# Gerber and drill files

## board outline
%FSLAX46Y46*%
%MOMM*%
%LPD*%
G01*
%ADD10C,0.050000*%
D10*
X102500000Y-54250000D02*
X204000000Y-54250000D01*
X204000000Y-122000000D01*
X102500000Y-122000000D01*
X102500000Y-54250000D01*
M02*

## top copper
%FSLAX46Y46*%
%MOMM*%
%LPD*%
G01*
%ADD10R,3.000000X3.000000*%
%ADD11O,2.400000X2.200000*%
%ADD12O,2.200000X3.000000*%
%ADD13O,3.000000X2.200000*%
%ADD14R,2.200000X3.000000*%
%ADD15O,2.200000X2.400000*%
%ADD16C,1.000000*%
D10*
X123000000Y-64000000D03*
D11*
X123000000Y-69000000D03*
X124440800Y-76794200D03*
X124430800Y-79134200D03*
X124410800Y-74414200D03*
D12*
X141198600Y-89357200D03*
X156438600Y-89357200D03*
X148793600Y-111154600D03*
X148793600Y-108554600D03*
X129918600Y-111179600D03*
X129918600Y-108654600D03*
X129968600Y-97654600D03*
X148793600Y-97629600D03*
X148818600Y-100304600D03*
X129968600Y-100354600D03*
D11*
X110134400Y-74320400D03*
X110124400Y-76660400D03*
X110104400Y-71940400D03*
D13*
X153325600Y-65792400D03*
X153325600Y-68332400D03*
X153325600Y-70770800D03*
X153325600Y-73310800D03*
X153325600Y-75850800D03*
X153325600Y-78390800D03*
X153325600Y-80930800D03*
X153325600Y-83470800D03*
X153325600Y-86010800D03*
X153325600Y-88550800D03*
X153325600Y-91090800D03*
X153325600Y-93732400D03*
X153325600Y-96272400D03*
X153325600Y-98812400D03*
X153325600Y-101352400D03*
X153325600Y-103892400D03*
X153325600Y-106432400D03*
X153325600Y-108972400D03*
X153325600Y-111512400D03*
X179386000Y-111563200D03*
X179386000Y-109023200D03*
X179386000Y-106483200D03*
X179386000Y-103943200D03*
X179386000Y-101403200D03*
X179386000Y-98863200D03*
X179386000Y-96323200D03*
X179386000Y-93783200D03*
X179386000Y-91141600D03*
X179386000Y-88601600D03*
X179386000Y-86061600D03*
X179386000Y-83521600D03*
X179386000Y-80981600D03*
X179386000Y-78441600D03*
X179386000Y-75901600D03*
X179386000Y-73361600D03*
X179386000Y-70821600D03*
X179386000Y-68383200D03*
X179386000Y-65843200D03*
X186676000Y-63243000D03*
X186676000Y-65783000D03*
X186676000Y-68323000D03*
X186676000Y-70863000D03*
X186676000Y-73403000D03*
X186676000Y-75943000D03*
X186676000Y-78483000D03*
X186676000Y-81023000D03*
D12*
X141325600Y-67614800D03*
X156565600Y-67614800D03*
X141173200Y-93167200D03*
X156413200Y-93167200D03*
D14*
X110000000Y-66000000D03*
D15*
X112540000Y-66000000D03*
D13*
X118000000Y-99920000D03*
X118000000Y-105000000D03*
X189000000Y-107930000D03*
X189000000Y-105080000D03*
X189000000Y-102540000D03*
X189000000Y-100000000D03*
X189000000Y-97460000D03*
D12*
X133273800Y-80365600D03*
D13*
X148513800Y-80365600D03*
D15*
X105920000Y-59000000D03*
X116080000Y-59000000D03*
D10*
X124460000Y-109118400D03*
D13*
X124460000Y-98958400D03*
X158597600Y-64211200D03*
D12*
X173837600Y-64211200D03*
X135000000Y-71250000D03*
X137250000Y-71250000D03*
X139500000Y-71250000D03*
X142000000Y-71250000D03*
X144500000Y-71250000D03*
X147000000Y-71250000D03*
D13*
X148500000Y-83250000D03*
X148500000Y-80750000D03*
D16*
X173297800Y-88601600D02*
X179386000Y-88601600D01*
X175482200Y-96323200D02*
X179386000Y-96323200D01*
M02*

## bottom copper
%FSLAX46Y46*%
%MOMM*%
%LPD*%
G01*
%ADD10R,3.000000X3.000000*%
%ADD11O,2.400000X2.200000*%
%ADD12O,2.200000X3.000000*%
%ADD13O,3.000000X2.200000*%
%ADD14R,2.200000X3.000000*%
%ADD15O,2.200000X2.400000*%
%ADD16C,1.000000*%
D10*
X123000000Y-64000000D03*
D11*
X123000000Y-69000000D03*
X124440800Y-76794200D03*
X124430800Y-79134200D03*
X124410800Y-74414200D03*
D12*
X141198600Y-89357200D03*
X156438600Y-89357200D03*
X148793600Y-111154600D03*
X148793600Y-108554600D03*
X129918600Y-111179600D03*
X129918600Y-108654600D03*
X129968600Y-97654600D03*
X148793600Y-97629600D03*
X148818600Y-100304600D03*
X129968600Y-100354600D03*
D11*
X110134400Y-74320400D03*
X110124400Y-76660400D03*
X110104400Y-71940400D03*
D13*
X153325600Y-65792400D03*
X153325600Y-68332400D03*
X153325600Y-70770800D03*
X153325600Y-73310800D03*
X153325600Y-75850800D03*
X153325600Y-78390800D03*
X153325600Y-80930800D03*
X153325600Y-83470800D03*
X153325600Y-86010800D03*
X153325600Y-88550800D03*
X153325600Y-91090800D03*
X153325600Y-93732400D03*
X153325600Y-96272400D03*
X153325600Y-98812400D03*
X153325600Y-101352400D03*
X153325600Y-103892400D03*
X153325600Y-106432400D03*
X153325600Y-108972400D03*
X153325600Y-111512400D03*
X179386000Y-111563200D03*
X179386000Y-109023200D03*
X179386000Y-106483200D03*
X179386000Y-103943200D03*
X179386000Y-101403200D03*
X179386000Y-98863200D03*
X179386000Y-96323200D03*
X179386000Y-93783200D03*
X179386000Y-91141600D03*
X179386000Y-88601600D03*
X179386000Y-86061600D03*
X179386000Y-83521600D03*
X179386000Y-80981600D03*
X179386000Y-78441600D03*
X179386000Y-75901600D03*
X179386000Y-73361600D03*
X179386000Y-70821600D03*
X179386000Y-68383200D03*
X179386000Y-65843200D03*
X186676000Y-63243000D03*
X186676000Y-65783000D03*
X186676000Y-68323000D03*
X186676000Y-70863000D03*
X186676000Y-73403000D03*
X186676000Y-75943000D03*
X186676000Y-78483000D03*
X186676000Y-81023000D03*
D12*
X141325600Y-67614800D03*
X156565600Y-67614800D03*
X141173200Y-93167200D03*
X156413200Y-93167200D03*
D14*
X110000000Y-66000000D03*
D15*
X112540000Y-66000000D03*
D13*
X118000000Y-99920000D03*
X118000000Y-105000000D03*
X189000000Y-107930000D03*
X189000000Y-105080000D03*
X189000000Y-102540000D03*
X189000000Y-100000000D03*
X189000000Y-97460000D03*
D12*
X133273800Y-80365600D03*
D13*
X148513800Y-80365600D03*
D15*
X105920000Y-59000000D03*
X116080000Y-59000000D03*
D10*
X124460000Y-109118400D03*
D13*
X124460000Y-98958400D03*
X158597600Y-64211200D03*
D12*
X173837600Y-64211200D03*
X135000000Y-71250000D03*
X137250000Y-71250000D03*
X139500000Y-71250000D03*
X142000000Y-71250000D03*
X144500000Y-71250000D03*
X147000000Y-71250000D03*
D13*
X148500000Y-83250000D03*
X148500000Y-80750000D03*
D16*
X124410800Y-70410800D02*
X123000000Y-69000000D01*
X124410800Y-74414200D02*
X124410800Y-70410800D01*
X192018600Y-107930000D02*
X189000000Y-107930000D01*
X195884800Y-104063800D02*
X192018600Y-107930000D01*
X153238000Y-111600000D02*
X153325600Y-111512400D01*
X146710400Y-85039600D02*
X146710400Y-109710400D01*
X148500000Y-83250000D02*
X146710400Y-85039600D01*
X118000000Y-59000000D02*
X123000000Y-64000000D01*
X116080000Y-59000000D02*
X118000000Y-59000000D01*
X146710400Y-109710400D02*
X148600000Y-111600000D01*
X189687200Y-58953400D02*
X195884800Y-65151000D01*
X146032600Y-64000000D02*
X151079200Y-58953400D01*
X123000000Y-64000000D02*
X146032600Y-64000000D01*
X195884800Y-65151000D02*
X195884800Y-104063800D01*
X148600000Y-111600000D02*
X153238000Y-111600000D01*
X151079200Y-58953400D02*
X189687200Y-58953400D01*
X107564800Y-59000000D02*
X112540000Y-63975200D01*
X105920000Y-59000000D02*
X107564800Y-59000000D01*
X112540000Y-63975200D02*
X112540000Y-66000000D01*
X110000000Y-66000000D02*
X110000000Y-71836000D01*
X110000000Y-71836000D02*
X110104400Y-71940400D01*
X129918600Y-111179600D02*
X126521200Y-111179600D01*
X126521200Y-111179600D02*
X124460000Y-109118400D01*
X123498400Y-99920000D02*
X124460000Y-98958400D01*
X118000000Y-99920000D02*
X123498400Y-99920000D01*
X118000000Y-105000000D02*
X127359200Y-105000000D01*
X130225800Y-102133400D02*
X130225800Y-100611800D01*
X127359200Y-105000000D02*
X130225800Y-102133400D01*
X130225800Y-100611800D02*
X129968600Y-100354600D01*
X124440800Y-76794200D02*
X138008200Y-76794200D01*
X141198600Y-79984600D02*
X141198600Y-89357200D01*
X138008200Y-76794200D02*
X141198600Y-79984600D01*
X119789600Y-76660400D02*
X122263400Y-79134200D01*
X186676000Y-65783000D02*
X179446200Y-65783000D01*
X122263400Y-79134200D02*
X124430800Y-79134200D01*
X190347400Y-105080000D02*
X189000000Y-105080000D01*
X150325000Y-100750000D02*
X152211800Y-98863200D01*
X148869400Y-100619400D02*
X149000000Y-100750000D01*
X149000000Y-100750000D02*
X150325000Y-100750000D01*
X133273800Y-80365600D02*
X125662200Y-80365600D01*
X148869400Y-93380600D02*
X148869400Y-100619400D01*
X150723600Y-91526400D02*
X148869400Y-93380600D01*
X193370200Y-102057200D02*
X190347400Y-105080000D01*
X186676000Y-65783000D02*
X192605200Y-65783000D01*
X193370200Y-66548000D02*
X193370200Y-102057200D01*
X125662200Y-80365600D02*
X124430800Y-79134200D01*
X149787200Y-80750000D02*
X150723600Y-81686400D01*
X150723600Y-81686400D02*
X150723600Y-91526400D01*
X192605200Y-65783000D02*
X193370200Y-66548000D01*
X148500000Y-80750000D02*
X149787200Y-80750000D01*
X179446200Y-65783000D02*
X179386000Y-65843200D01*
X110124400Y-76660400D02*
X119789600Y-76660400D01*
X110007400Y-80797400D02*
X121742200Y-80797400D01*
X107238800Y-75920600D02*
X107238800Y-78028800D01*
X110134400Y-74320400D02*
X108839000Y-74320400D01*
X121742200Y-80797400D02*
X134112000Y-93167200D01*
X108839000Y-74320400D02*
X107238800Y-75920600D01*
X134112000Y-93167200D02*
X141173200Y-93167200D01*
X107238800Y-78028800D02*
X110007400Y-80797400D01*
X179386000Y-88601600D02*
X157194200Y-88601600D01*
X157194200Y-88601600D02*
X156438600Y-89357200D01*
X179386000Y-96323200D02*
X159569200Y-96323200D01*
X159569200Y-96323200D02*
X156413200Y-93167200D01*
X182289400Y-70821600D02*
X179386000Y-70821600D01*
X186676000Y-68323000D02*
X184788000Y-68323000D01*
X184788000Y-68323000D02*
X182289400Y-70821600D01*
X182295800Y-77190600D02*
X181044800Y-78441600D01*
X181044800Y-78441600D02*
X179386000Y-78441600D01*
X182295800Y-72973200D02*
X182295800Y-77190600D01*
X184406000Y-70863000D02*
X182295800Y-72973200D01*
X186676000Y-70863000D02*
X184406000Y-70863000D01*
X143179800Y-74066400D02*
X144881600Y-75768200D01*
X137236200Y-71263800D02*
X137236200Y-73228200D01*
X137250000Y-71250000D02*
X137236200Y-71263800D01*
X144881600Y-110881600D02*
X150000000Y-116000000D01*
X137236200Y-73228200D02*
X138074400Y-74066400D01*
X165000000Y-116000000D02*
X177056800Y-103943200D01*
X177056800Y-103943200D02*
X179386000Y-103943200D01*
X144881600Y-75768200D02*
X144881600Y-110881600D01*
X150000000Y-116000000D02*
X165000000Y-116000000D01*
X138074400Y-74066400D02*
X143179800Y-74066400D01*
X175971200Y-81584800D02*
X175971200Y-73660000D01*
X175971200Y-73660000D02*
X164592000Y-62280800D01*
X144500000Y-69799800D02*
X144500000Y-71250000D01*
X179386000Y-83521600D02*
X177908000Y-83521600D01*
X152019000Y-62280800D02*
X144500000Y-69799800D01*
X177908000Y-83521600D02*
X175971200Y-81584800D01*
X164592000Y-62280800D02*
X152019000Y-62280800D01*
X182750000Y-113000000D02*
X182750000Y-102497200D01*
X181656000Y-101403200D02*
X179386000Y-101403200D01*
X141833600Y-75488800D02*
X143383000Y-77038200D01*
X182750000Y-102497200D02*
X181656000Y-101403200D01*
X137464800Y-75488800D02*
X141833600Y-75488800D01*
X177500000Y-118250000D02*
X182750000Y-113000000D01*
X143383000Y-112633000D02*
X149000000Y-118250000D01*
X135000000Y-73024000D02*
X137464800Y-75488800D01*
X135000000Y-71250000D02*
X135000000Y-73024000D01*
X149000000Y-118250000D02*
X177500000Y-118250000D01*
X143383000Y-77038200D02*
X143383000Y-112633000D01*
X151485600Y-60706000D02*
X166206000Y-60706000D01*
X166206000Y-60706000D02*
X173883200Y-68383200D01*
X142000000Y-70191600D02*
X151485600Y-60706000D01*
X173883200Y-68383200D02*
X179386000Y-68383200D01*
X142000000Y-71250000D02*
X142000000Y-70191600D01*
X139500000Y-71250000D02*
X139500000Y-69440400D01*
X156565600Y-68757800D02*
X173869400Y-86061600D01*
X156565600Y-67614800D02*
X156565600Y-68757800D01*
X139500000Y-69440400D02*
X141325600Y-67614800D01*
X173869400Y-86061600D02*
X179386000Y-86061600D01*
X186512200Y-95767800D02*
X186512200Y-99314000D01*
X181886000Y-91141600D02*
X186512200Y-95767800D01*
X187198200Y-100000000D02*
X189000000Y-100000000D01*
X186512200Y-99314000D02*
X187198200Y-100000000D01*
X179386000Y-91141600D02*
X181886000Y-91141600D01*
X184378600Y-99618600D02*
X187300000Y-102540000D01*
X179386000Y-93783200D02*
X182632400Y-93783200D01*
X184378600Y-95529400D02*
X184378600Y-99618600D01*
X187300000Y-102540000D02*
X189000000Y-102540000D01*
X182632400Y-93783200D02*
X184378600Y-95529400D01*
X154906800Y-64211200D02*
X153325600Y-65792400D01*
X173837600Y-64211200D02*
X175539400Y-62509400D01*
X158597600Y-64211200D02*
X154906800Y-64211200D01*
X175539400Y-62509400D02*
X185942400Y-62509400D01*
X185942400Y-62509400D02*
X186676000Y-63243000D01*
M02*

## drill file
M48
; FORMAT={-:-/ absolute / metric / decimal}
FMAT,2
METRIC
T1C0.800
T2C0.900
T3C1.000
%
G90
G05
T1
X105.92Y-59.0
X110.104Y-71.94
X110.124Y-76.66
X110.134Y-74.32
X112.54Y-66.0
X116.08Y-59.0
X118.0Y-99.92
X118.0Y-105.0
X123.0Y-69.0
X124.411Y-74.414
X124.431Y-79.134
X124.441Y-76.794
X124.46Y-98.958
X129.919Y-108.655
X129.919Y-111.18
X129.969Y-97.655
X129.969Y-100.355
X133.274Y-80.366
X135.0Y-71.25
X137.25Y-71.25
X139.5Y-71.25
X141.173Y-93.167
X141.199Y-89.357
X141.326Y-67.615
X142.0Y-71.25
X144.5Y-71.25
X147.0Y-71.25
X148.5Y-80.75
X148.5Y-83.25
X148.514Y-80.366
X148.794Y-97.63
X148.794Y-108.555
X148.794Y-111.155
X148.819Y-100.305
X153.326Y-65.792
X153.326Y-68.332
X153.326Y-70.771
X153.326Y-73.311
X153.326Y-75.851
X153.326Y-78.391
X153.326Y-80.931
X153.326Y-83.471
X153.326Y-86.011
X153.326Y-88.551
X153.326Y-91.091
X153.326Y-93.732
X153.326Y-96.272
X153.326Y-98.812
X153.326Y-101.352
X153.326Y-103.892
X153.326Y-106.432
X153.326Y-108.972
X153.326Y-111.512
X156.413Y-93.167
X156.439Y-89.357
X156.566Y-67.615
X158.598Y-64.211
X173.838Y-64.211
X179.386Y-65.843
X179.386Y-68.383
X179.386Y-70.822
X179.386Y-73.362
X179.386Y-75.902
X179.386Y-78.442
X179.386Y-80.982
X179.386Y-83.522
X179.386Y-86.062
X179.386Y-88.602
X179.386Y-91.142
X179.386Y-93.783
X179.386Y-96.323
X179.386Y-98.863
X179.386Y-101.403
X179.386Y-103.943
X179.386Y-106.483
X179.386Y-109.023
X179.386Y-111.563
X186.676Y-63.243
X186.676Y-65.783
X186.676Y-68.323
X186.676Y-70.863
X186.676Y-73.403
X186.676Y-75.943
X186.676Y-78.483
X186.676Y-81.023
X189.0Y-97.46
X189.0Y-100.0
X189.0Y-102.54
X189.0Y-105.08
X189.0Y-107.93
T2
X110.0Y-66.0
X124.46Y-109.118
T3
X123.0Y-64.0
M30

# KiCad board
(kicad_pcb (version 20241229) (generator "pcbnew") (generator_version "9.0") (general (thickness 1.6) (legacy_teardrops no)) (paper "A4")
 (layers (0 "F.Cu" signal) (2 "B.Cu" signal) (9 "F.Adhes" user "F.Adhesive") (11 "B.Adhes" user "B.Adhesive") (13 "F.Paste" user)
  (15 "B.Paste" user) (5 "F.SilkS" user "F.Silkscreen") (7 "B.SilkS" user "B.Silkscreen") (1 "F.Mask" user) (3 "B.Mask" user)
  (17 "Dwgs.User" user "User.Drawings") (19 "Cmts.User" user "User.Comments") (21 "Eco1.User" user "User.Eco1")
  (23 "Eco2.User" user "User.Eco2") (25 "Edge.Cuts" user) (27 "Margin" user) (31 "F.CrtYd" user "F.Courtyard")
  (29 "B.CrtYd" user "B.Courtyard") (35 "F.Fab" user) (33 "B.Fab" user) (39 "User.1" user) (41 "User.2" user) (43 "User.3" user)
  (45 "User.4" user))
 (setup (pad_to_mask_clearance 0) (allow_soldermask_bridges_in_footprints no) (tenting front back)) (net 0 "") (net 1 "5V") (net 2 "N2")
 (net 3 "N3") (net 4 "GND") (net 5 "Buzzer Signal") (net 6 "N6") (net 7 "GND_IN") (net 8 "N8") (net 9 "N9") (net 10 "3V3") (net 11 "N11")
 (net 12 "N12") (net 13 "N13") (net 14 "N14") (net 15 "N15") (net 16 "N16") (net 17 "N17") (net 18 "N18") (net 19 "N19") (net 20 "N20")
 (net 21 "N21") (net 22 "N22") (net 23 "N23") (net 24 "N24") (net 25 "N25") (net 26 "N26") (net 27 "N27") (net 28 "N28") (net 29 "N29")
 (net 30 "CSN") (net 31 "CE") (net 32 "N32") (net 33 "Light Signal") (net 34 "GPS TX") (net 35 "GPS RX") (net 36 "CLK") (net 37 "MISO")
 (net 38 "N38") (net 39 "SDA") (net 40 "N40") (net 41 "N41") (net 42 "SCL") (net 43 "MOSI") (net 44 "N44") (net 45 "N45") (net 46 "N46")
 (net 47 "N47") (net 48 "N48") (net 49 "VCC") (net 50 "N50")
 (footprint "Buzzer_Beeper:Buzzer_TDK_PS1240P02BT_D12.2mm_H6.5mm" (layer "F.Cu") (at 123 64 -90)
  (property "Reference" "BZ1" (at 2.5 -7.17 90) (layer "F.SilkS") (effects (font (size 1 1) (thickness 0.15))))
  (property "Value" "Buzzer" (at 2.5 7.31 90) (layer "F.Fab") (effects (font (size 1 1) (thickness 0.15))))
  (pad "1" thru_hole rect (at 0 0 270) (size 3 3) (drill 1) (layers "*.Cu" "*.Mask") (remove_unused_layers no) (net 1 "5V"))
  (pad "2" thru_hole oval (at 5 0) (size 2.4 2.2) (drill 0.8) (layers "*.Cu" "*.Mask") (remove_unused_layers no) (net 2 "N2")
   (thermal_bridge_angle 45)))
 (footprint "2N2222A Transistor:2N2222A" (layer "F.Cu") (at 125.7808 76.7842 -90)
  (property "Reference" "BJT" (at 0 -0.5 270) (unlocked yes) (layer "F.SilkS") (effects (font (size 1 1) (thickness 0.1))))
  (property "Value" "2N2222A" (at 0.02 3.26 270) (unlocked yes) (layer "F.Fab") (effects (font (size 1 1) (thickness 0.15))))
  (pad "1" thru_hole oval (at 0.01 1.34) (size 2.4 2.2) (drill 0.8) (layers "*.Cu" "*.Mask") (remove_unused_layers no) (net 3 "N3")
   (thermal_bridge_angle 45))
  (pad "2" thru_hole oval (at 2.35 1.35) (size 2.4 2.2) (drill 0.8) (layers "*.Cu" "*.Mask") (remove_unused_layers no) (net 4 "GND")
   (thermal_bridge_angle 45))
  (pad "3" thru_hole oval (at -2.37 1.37) (size 2.4 2.2) (drill 0.8) (layers "*.Cu" "*.Mask") (remove_unused_layers no) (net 2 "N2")
   (thermal_bridge_angle 45)))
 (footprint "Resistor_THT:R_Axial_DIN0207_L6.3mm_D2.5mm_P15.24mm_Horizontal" (layer "F.Cu") (at 141.1986 89.3572)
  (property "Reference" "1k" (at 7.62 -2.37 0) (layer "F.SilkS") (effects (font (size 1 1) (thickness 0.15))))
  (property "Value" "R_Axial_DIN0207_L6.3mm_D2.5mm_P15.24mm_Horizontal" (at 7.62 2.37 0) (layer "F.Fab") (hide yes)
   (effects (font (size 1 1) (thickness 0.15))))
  (pad "1" thru_hole oval (at 0 0) (size 2.2 3) (drill 0.8) (layers "*.Cu" "*.Mask") (remove_unused_layers no) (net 3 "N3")
   (thermal_bridge_angle 45))
  (pad "2" thru_hole oval (at 15.24 0) (size 2.2 3) (drill 0.8) (layers "*.Cu" "*.Mask") (remove_unused_layers no) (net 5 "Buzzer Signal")
   (thermal_bridge_angle 45)))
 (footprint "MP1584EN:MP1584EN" (layer "F.Cu") (at 150.8936 113.4546 180)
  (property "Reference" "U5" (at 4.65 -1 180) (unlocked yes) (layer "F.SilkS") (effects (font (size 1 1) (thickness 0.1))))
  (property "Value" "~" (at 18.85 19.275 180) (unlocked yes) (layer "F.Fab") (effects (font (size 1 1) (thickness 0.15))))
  (pad "1" thru_hole oval (at 2.1 2.3 180) (size 2.2 3) (drill 0.8) (layers "*.Cu" "*.Mask") (remove_unused_layers no) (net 1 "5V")
   (thermal_bridge_angle 45))
  (pad "2" thru_hole oval (at 2.1 4.9 180) (size 2.2 3) (drill 0.8) (layers "*.Cu" "*.Mask") (remove_unused_layers no)
   (thermal_bridge_angle 45))
  (pad "3" thru_hole oval (at 20.975 2.275 180) (size 2.2 3) (drill 0.8) (layers "*.Cu" "*.Mask") (remove_unused_layers no) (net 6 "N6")
   (thermal_bridge_angle 45))
  (pad "4" thru_hole oval (at 20.975 4.8 180) (size 2.2 3) (drill 0.8) (layers "*.Cu" "*.Mask") (remove_unused_layers no)
   (thermal_bridge_angle 45))
  (pad "5" thru_hole oval (at 20.925 15.8 180) (size 2.2 3) (drill 0.8) (layers "*.Cu" "*.Mask") (remove_unused_layers no)
   (thermal_bridge_angle 45))
  (pad "6" thru_hole oval (at 2.1 15.825 180) (size 2.2 3) (drill 0.8) (layers "*.Cu" "*.Mask") (remove_unused_layers no)
   (thermal_bridge_angle 45))
  (pad "7" thru_hole oval (at 2.075 13.15 180) (size 2.2 3) (drill 0.8) (layers "*.Cu" "*.Mask") (remove_unused_layers no) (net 4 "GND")
   (thermal_bridge_angle 45))
  (pad "8" thru_hole oval (at 20.925 13.1 180) (size 2.2 3) (drill 0.8) (layers "*.Cu" "*.Mask") (remove_unused_layers no) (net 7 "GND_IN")
   (thermal_bridge_angle 45)))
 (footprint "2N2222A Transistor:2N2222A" (layer "F.Cu") (at 111.4744 74.3104 -90)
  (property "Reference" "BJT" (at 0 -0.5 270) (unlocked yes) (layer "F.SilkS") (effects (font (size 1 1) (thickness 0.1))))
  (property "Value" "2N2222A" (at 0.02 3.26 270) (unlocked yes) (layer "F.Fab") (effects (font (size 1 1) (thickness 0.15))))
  (pad "1" thru_hole oval (at 0.01 1.34) (size 2.4 2.2) (drill 0.8) (layers "*.Cu" "*.Mask") (remove_unused_layers no) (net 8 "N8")
   (thermal_bridge_angle 45))
  (pad "2" thru_hole oval (at 2.35 1.35) (size 2.4 2.2) (drill 0.8) (layers "*.Cu" "*.Mask") (remove_unused_layers no) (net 4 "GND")
   (thermal_bridge_angle 45))
  (pad "3" thru_hole oval (at -2.37 1.37) (size 2.4 2.2) (drill 0.8) (layers "*.Cu" "*.Mask") (remove_unused_layers no) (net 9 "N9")
   (thermal_bridge_angle 45)))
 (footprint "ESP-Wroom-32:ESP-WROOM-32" (layer "F.Cu") (at 153.986 61.4236)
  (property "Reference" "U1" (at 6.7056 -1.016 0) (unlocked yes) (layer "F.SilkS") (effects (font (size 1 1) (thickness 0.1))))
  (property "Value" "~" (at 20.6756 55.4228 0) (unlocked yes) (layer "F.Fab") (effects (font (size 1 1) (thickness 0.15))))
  (pad "1" thru_hole oval (at -0.6604 4.3688) (size 3 2.2) (drill 0.8) (layers "*.Cu" "*.Mask") (remove_unused_layers no) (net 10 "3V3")
   (thermal_bridge_angle 45))
  (pad "2" thru_hole oval (at -0.6604 6.9088) (size 3 2.2) (drill 0.8) (layers "*.Cu" "*.Mask") (remove_unused_layers no) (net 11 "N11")
   (thermal_bridge_angle 45))
  (pad "3" thru_hole oval (at -0.6604 9.3472) (size 3 2.2) (drill 0.8) (layers "*.Cu" "*.Mask") (remove_unused_layers no) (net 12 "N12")
   (thermal_bridge_angle 45))
  (pad "4" thru_hole oval (at -0.6604 11.8872) (size 3 2.2) (drill 0.8) (layers "*.Cu" "*.Mask") (remove_unused_layers no) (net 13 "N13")
   (thermal_bridge_angle 45))
  (pad "5" thru_hole oval (at -0.6604 14.4272) (size 3 2.2) (drill 0.8) (layers "*.Cu" "*.Mask") (remove_unused_layers no) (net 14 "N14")
   (thermal_bridge_angle 45))
  (pad "6" thru_hole oval (at -0.6604 16.9672) (size 3 2.2) (drill 0.8) (layers "*.Cu" "*.Mask") (remove_unused_layers no) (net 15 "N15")
   (thermal_bridge_angle 45))
  (pad "7" thru_hole oval (at -0.6604 19.5072) (size 3 2.2) (drill 0.8) (layers "*.Cu" "*.Mask") (remove_unused_layers no) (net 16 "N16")
   (thermal_bridge_angle 45))
  (pad "8" thru_hole oval (at -0.6604 22.0472) (size 3 2.2) (drill 0.8) (layers "*.Cu" "*.Mask") (remove_unused_layers no) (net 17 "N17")
   (thermal_bridge_angle 45))
  (pad "9" thru_hole oval (at -0.6604 24.5872) (size 3 2.2) (drill 0.8) (layers "*.Cu" "*.Mask") (remove_unused_layers no) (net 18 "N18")
   (thermal_bridge_angle 45))
  (pad "10" thru_hole oval (at -0.6604 27.1272) (size 3 2.2) (drill 0.8) (layers "*.Cu" "*.Mask") (remove_unused_layers no) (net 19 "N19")
   (thermal_bridge_angle 45))
  (pad "11" thru_hole oval (at -0.6604 29.6672) (size 3 2.2) (drill 0.8) (layers "*.Cu" "*.Mask") (remove_unused_layers no) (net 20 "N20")
   (thermal_bridge_angle 45))
  (pad "12" thru_hole oval (at -0.6604 32.3088) (size 3 2.2) (drill 0.8) (layers "*.Cu" "*.Mask") (remove_unused_layers no) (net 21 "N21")
   (thermal_bridge_angle 45))
  (pad "13" thru_hole oval (at -0.6604 34.8488) (size 3 2.2) (drill 0.8) (layers "*.Cu" "*.Mask") (remove_unused_layers no) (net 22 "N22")
   (thermal_bridge_angle 45))
  (pad "14" thru_hole oval (at -0.6604 37.3888) (size 3 2.2) (drill 0.8) (layers "*.Cu" "*.Mask") (remove_unused_layers no) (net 4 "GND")
   (thermal_bridge_angle 45))
  (pad "15" thru_hole oval (at -0.6604 39.9288) (size 3 2.2) (drill 0.8) (layers "*.Cu" "*.Mask") (remove_unused_layers no) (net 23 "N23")
   (thermal_bridge_angle 45))
  (pad "16" thru_hole oval (at -0.6604 42.4688) (size 3 2.2) (drill 0.8) (layers "*.Cu" "*.Mask") (remove_unused_layers no) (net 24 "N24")
   (thermal_bridge_angle 45))
  (pad "17" thru_hole oval (at -0.6604 45.0088) (size 3 2.2) (drill 0.8) (layers "*.Cu" "*.Mask") (remove_unused_layers no) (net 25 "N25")
   (thermal_bridge_angle 45))
  (pad "18" thru_hole oval (at -0.6604 47.5488) (size 3 2.2) (drill 0.8) (layers "*.Cu" "*.Mask") (remove_unused_layers no) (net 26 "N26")
   (thermal_bridge_angle 45))
  (pad "19" thru_hole oval (at -0.6604 50.0888) (size 3 2.2) (drill 0.8) (layers "*.Cu" "*.Mask") (remove_unused_layers no) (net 1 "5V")
   (thermal_bridge_angle 45))
  (pad "20" thru_hole oval (at 25.4 50.1396) (size 3 2.2) (drill 0.8) (layers "*.Cu" "*.Mask") (remove_unused_layers no) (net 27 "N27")
   (thermal_bridge_angle 45))
  (pad "21" thru_hole oval (at 25.4 47.5996) (size 3 2.2) (drill 0.8) (layers "*.Cu" "*.Mask") (remove_unused_layers no) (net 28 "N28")
   (thermal_bridge_angle 45))
  (pad "22" thru_hole oval (at 25.4 45.0596) (size 3 2.2) (drill 0.8) (layers "*.Cu" "*.Mask") (remove_unused_layers no) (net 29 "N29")
   (thermal_bridge_angle 45))
  (pad "23" thru_hole oval (at 25.4 42.5196) (size 3 2.2) (drill 0.8) (layers "*.Cu" "*.Mask") (remove_unused_layers no) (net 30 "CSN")
   (thermal_bridge_angle 45))
  (pad "24" thru_hole oval (at 25.4 39.9796) (size 3 2.2) (drill 0.8) (layers "*.Cu" "*.Mask") (remove_unused_layers no) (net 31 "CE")
   (thermal_bridge_angle 45))
  (pad "25" thru_hole oval (at 25.4 37.4396) (size 3 2.2) (drill 0.8) (layers "*.Cu" "*.Mask") (remove_unused_layers no) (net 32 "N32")
   (thermal_bridge_angle 45))
  (pad "26" thru_hole oval (at 25.4 34.8996) (size 3 2.2) (drill 0.8) (layers "*.Cu" "*.Mask") (remove_unused_layers no)
   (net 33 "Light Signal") (thermal_bridge_angle 45))
  (pad "27" thru_hole oval (at 25.4 32.3596) (size 3 2.2) (drill 0.8) (layers "*.Cu" "*.Mask") (remove_unused_layers no) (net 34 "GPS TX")
   (thermal_bridge_angle 45))
  (pad "28" thru_hole oval (at 25.4 29.718) (size 3 2.2) (drill 0.8) (layers "*.Cu" "*.Mask") (remove_unused_layers no) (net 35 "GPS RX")
   (thermal_bridge_angle 45))
  (pad "29" thru_hole oval (at 25.4 27.178) (size 3 2.2) (drill 0.8) (layers "*.Cu" "*.Mask") (remove_unused_layers no)
   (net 5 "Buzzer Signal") (thermal_bridge_angle 45))
  (pad "30" thru_hole oval (at 25.4 24.638) (size 3 2.2) (drill 0.8) (layers "*.Cu" "*.Mask") (remove_unused_layers no) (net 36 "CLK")
   (thermal_bridge_angle 45))
  (pad "31" thru_hole oval (at 25.4 22.098) (size 3 2.2) (drill 0.8) (layers "*.Cu" "*.Mask") (remove_unused_layers no) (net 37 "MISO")
   (thermal_bridge_angle 45))
  (pad "32" thru_hole oval (at 25.4 19.558) (size 3 2.2) (drill 0.8) (layers "*.Cu" "*.Mask") (remove_unused_layers no) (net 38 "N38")
   (thermal_bridge_angle 45))
  (pad "33" thru_hole oval (at 25.4 17.018) (size 3 2.2) (drill 0.8) (layers "*.Cu" "*.Mask") (remove_unused_layers no) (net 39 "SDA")
   (thermal_bridge_angle 45))
  (pad "34" thru_hole oval (at 25.4 14.478) (size 3 2.2) (drill 0.8) (layers "*.Cu" "*.Mask") (remove_unused_layers no) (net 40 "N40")
   (thermal_bridge_angle 45))
  (pad "35" thru_hole oval (at 25.4 11.938) (size 3 2.2) (drill 0.8) (layers "*.Cu" "*.Mask") (remove_unused_layers no) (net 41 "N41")
   (thermal_bridge_angle 45))
  (pad "36" thru_hole oval (at 25.4 9.398) (size 3 2.2) (drill 0.8) (layers "*.Cu" "*.Mask") (remove_unused_layers no) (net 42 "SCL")
   (thermal_bridge_angle 45))
  (pad "37" thru_hole oval (at 25.4 6.9596) (size 3 2.2) (drill 0.8) (layers "*.Cu" "*.Mask") (remove_unused_layers no) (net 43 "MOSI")
   (thermal_bridge_angle 45))
  (pad "38" thru_hole oval (at 25.4 4.4196) (size 3 2.2) (drill 0.8) (layers "*.Cu" "*.Mask") (remove_unused_layers no) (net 4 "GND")
   (thermal_bridge_angle 45)))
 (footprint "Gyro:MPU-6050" (layer "F.Cu") (at 200.9 61.719 -90)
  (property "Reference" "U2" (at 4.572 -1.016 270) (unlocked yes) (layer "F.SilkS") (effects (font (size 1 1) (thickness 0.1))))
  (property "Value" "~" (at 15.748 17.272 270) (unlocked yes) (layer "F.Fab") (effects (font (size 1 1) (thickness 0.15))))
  (pad "1" thru_hole oval (at 1.524 14.224 270) (size 2.2 3) (drill 0.8) (layers "*.Cu" "*.Mask") (remove_unused_layers no) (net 10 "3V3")
   (thermal_bridge_angle 45))
  (pad "2" thru_hole oval (at 4.064 14.224 270) (size 2.2 3) (drill 0.8) (layers "*.Cu" "*.Mask") (remove_unused_layers no) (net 4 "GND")
   (thermal_bridge_angle 45))
  (pad "3" thru_hole oval (at 6.604 14.224 270) (size 2.2 3) (drill 0.8) (layers "*.Cu" "*.Mask") (remove_unused_layers no) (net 42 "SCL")
   (thermal_bridge_angle 45))
  (pad "4" thru_hole oval (at 9.144 14.224 270) (size 2.2 3) (drill 0.8) (layers "*.Cu" "*.Mask") (remove_unused_layers no) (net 39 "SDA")
   (thermal_bridge_angle 45))
  (pad "5" thru_hole oval (at 11.684 14.224 270) (size 2.2 3) (drill 0.8) (layers "*.Cu" "*.Mask") (remove_unused_layers no) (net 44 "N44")
   (thermal_bridge_angle 45))
  (pad "6" thru_hole oval (at 14.224 14.224 270) (size 2.2 3) (drill 0.8) (layers "*.Cu" "*.Mask") (remove_unused_layers no) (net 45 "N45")
   (thermal_bridge_angle 45))
  (pad "7" thru_hole oval (at 16.764 14.224 270) (size 2.2 3) (drill 0.8) (layers "*.Cu" "*.Mask") (remove_unused_layers no) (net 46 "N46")
   (thermal_bridge_angle 45))
  (pad "8" thru_hole oval (at 19.304 14.224 270) (size 2.2 3) (drill 0.8) (layers "*.Cu" "*.Mask") (remove_unused_layers no) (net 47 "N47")
   (thermal_bridge_angle 45)))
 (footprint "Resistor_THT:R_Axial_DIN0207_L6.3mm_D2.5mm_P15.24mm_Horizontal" (layer "F.Cu") (at 141.3256 67.6148)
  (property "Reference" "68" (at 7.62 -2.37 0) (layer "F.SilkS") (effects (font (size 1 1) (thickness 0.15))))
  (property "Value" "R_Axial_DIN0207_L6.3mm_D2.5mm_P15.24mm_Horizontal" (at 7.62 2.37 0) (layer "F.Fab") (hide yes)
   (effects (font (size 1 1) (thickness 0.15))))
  (pad "1" thru_hole oval (at 0 0) (size 2.2 3) (drill 0.8) (layers "*.Cu" "*.Mask") (remove_unused_layers no) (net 36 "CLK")
   (thermal_bridge_angle 45))
  (pad "2" thru_hole oval (at 15.24 0) (size 2.2 3) (drill 0.8) (layers "*.Cu" "*.Mask") (remove_unused_layers no) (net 36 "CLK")
   (thermal_bridge_angle 45)))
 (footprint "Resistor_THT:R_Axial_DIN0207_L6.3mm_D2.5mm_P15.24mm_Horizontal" (layer "F.Cu") (at 141.1732 93.1672)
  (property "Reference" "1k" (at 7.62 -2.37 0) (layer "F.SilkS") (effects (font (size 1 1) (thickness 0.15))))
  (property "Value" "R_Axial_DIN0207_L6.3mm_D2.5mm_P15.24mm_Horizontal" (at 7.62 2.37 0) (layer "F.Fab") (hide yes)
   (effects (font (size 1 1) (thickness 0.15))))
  (pad "1" thru_hole oval (at 0 0) (size 2.2 3) (drill 0.8) (layers "*.Cu" "*.Mask") (remove_unused_layers no) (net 8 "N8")
   (thermal_bridge_angle 45))
  (pad "2" thru_hole oval (at 15.24 0) (size 2.2 3) (drill 0.8) (layers "*.Cu" "*.Mask") (remove_unused_layers no) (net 33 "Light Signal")
   (thermal_bridge_angle 45)))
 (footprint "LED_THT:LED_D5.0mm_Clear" (layer "F.Cu") (at 110 66)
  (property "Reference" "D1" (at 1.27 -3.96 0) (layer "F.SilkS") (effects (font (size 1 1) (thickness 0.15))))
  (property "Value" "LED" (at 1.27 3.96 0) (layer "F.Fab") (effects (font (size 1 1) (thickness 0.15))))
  (pad "1" thru_hole rect (at 0 0) (size 2.2 3) (drill 0.9) (layers "*.Cu" "*.Mask") (remove_unused_layers no) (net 9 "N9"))
  (pad "2" thru_hole oval (at 2.54 0 90) (size 2.4 2.2) (drill 0.8) (layers "*.Cu" "*.Mask") (remove_unused_layers no) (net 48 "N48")
   (thermal_bridge_angle 45)))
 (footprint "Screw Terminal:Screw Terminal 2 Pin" (layer "F.Cu") (at 121.85 97.38 -90)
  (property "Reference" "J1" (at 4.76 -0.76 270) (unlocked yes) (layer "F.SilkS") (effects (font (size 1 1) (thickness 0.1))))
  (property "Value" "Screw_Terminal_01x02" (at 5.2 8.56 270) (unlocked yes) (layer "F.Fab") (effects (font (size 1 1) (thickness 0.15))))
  (pad "1" thru_hole oval (at 2.54 3.85 270) (size 2.2 3) (drill 0.8) (layers "*.Cu" "*.Mask") (remove_unused_layers no) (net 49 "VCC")
   (thermal_bridge_angle 45))
  (pad "2" thru_hole oval (at 7.62 3.85 270) (size 2.2 3) (drill 0.8) (layers "*.Cu" "*.Mask") (remove_unused_layers no) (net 7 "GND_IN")
   (thermal_bridge_angle 45)))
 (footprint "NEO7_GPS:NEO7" (layer "F.Cu") (at 239.419 115.748 180)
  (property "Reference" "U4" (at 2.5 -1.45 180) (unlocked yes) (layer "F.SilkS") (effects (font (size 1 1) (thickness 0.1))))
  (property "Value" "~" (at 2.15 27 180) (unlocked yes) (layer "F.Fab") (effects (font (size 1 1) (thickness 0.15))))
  (pad "1" thru_hole oval (at 50.419 7.818 180) (size 3 2.2) (drill 0.8) (layers "*.Cu" "*.Mask") (remove_unused_layers no) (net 1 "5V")
   (thermal_bridge_angle 45))
  (pad "2" thru_hole oval (at 50.419 10.668 180) (size 3 2.2) (drill 0.8) (layers "*.Cu" "*.Mask") (remove_unused_layers no) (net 4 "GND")
   (thermal_bridge_angle 45))
  (pad "3" thru_hole oval (at 50.419 13.208 180) (size 3 2.2) (drill 0.8) (layers "*.Cu" "*.Mask") (remove_unused_layers no)
   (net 34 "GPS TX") (thermal_bridge_angle 45))
  (pad "4" thru_hole oval (at 50.419 15.748 180) (size 3 2.2) (drill 0.8) (layers "*.Cu" "*.Mask") (remove_unused_layers no)
   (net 35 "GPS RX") (thermal_bridge_angle 45))
  (pad "5" thru_hole oval (at 50.419 18.288 180) (size 3 2.2) (drill 0.8) (layers "*.Cu" "*.Mask") (remove_unused_layers no)
   (thermal_bridge_angle 45)))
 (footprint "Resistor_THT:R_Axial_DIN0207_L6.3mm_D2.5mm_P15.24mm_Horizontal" (layer "F.Cu") (at 133.2738 80.3656)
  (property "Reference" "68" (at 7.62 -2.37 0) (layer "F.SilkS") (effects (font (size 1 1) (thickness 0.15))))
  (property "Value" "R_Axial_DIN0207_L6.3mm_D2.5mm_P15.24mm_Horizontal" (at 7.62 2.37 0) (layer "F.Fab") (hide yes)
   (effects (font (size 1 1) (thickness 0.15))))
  (pad "1" thru_hole oval (at 0 0) (size 2.2 3) (drill 0.8) (layers "*.Cu" "*.Mask") (remove_unused_layers no) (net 4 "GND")
   (thermal_bridge_angle 45))
  (pad "2" thru_hole oval (at 15.24 0) (size 3 2.2) (drill 0.8) (layers "*.Cu" "*.Mask") (remove_unused_layers no) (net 4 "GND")
   (thermal_bridge_angle 45)))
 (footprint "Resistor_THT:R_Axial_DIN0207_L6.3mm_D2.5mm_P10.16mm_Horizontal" (layer "F.Cu") (at 105.92 59)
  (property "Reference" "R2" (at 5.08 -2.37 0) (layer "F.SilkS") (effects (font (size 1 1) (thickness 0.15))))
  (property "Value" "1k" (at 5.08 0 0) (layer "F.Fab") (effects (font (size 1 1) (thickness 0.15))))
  (pad "1" thru_hole oval (at 0 0 90) (size 2.4 2.2) (drill 0.8) (layers "*.Cu" "*.Mask") (remove_unused_layers no) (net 48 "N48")
   (thermal_bridge_angle 45))
  (pad "2" thru_hole oval (at 10.16 0 90) (size 2.4 2.2) (drill 0.8) (layers "*.Cu" "*.Mask") (remove_unused_layers no) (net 1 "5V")
   (thermal_bridge_angle 45)))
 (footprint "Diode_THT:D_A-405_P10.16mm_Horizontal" (layer "F.Cu") (at 124.46 109.1184 90)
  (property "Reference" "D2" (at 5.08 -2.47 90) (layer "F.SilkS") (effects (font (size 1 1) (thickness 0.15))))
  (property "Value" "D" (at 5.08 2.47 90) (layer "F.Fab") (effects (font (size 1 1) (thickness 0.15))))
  (pad "1" thru_hole rect (at 0 0 90) (size 3 3) (drill 0.9) (layers "*.Cu" "*.Mask") (remove_unused_layers no) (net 6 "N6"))
  (pad "2" thru_hole oval (at 10.16 0 90) (size 2.2 3) (drill 0.8) (layers "*.Cu" "*.Mask") (remove_unused_layers no) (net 49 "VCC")
   (thermal_bridge_angle 45)))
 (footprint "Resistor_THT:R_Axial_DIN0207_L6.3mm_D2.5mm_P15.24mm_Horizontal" (layer "F.Cu") (at 158.5976 64.2112)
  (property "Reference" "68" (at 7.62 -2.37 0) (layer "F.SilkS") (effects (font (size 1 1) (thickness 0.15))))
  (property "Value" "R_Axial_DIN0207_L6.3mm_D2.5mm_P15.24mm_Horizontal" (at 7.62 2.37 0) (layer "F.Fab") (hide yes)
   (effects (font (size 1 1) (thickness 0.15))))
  (pad "1" thru_hole oval (at 0 0) (size 3 2.2) (drill 0.8) (layers "*.Cu" "*.Mask") (remove_unused_layers no) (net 10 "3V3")
   (thermal_bridge_angle 45))
  (pad "2" thru_hole oval (at 15.24 0) (size 2.2 3) (drill 0.8) (layers "*.Cu" "*.Mask") (remove_unused_layers no) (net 10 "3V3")
   (thermal_bridge_angle 45)))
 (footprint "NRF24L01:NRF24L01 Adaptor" (layer "F.Cu") (at 141 74.5 90)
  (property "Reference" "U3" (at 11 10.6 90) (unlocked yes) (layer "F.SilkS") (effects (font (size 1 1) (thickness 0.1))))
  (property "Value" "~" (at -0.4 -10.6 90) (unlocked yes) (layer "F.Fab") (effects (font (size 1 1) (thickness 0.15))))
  (pad "1" thru_hole oval (at 3.25 -6 90) (size 3 2.2) (drill 0.8) (layers "*.Cu" "*.Mask") (remove_unused_layers no) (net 31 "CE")
   (thermal_bridge_angle 45))
  (pad "2" thru_hole oval (at 3.25 -3.75 90) (size 3 2.2) (drill 0.8) (layers "*.Cu" "*.Mask") (remove_unused_layers no) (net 30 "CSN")
   (thermal_bridge_angle 45))
  (pad "3" thru_hole oval (at 3.25 -1.5 90) (size 3 2.2) (drill 0.8) (layers "*.Cu" "*.Mask") (remove_unused_layers no) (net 36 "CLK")
   (thermal_bridge_angle 45))
  (pad "4" thru_hole oval (at 3.25 1 90) (size 3 2.2) (drill 0.8) (layers "*.Cu" "*.Mask") (remove_unused_layers no) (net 43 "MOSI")
   (thermal_bridge_angle 45))
  (pad "5" thru_hole oval (at 3.25 3.5 90) (size 3 2.2) (drill 0.8) (layers "*.Cu" "*.Mask") (remove_unused_layers no) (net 37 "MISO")
   (thermal_bridge_angle 45))
  (pad "6" thru_hole oval (at 3.25 6 90) (size 3 2.2) (drill 0.8) (layers "*.Cu" "*.Mask") (remove_unused_layers no) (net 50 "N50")
   (thermal_bridge_angle 45))
  (pad "7" thru_hole oval (at -8.75 7.5 90) (size 2.2 3) (drill 0.8) (layers "*.Cu" "*.Mask") (remove_unused_layers no) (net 1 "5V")
   (thermal_bridge_angle 45))
  (pad "8" thru_hole oval (at -6.25 7.5 90) (size 2.2 3) (drill 0.8) (layers "*.Cu" "*.Mask") (remove_unused_layers no) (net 4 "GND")
   (thermal_bridge_angle 45))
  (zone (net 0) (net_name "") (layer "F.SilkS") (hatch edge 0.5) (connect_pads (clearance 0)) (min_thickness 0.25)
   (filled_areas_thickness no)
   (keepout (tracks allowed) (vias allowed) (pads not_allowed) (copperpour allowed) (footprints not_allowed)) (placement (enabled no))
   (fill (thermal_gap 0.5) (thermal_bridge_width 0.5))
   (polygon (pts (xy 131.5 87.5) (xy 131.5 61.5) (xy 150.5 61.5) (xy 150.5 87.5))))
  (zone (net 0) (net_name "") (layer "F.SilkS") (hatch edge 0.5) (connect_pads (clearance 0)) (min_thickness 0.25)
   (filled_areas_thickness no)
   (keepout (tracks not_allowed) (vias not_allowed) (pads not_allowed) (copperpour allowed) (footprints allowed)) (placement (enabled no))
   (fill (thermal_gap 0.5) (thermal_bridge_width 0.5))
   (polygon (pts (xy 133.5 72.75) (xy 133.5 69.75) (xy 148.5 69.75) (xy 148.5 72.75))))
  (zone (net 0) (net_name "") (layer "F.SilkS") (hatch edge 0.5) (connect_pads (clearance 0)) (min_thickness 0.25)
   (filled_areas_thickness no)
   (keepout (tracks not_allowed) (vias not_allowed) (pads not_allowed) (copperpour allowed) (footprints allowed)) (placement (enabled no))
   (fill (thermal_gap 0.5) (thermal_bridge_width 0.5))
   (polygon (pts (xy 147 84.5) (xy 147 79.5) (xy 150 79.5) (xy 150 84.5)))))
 (gr_rect (start 102.5 54.25) (end 204 122) (stroke (width 0.05) (type default)) (fill no) (layer "Edge.Cuts"))
 (segment (start 124.4108 70.4108) (end 123 69) (width 1) (layer "B.Cu") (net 2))
 (segment (start 124.4108 74.4142) (end 124.4108 70.4108) (width 1) (layer "B.Cu") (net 2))
 (segment (start 192.0186 107.93) (end 189 107.93) (width 1) (layer "B.Cu") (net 1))
 (segment (start 195.8848 104.0638) (end 192.0186 107.93) (width 1) (layer "B.Cu") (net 1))
 (segment (start 153.238 111.6) (end 153.3256 111.5124) (width 1) (layer "B.Cu") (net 1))
 (segment (start 146.7104 85.0396) (end 146.7104 109.7104) (width 1) (layer "B.Cu") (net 1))
 (segment (start 148.5 83.25) (end 146.7104 85.0396) (width 1) (layer "B.Cu") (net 1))
 (segment (start 118 59) (end 123 64) (width 1) (layer "B.Cu") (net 1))
 (segment (start 116.08 59) (end 118 59) (width 1) (layer "B.Cu") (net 1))
 (segment (start 146.7104 109.7104) (end 148.6 111.6) (width 1) (layer "B.Cu") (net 1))
 (segment (start 189.6872 58.9534) (end 195.8848 65.151) (width 1) (layer "B.Cu") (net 1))
 (segment (start 146.0326 64) (end 151.0792 58.9534) (width 1) (layer "B.Cu") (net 1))
 (segment (start 123 64) (end 146.0326 64) (width 1) (layer "B.Cu") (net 1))
 (segment (start 195.8848 65.151) (end 195.8848 104.0638) (width 1) (layer "B.Cu") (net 1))
 (segment (start 148.6 111.6) (end 153.238 111.6) (width 1) (layer "B.Cu") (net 1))
 (segment (start 151.0792 58.9534) (end 189.6872 58.9534) (width 1) (layer "B.Cu") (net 1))
 (segment (start 107.5648 59) (end 112.54 63.9752) (width 1) (layer "B.Cu") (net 48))
 (segment (start 105.92 59) (end 107.5648 59) (width 1) (layer "B.Cu") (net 48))
 (segment (start 112.54 63.9752) (end 112.54 66) (width 1) (layer "B.Cu") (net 48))
 (segment (start 110 66) (end 110 71.836) (width 1) (layer "B.Cu") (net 9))
 (segment (start 110 71.836) (end 110.1044 71.9404) (width 1) (layer "B.Cu") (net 9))
 (segment (start 129.9186 111.1796) (end 126.5212 111.1796) (width 1) (layer "B.Cu") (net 6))
 (segment (start 126.5212 111.1796) (end 124.46 109.1184) (width 1) (layer "B.Cu") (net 6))
 (segment (start 123.4984 99.92) (end 124.46 98.9584) (width 1) (layer "B.Cu") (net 49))
 (segment (start 118 99.92) (end 123.4984 99.92) (width 1) (layer "B.Cu") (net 49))
 (segment (start 118 105) (end 127.3592 105) (width 1) (layer "B.Cu") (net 7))
 (segment (start 130.2258 102.1334) (end 130.2258 100.6118) (width 1) (layer "B.Cu") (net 7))
 (segment (start 127.3592 105) (end 130.2258 102.1334) (width 1) (layer "B.Cu") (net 7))
 (segment (start 130.2258 100.6118) (end 129.9686 100.3546) (width 1) (layer "B.Cu") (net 7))
 (segment (start 124.4408 76.7942) (end 138.0082 76.7942) (width 1) (layer "B.Cu") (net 3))
 (segment (start 141.1986 79.9846) (end 141.1986 89.3572) (width 1) (layer "B.Cu") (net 3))
 (segment (start 138.0082 76.7942) (end 141.1986 79.9846) (width 1) (layer "B.Cu") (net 3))
 (segment (start 119.7896 76.6604) (end 122.2634 79.1342) (width 1) (layer "B.Cu") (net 4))
 (segment (start 186.676 65.783) (end 179.4462 65.783) (width 1) (layer "B.Cu") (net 4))
 (segment (start 122.2634 79.1342) (end 124.4308 79.1342) (width 1) (layer "B.Cu") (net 4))
 (segment (start 190.3474 105.08) (end 189 105.08) (width 1) (layer "B.Cu") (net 4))
 (segment (start 150.325 100.75) (end 152.2118 98.8632) (width 1) (layer "B.Cu") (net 4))
 (segment (start 148.8694 100.6194) (end 149 100.75) (width 1) (layer "B.Cu") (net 4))
 (segment (start 149 100.75) (end 150.325 100.75) (width 1) (layer "B.Cu") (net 4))
 (segment (start 133.2738 80.3656) (end 125.6622 80.3656) (width 1) (layer "B.Cu") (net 4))
 (segment (start 148.8694 93.3806) (end 148.8694 100.6194) (width 1) (layer "B.Cu") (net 4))
 (segment (start 150.7236 91.5264) (end 148.8694 93.3806) (width 1) (layer "B.Cu") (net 4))
 (segment (start 193.3702 102.0572) (end 190.3474 105.08) (width 1) (layer "B.Cu") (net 4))
 (segment (start 186.676 65.783) (end 192.6052 65.783) (width 1) (layer "B.Cu") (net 4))
 (segment (start 193.3702 66.548) (end 193.3702 102.0572) (width 1) (layer "B.Cu") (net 4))
 (segment (start 125.6622 80.3656) (end 124.4308 79.1342) (width 1) (layer "B.Cu") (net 4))
 (segment (start 149.7872 80.75) (end 150.7236 81.6864) (width 1) (layer "B.Cu") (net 4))
 (segment (start 150.7236 81.6864) (end 150.7236 91.5264) (width 1) (layer "B.Cu") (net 4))
 (segment (start 192.6052 65.783) (end 193.3702 66.548) (width 1) (layer "B.Cu") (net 4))
 (segment (start 148.5 80.75) (end 149.7872 80.75) (width 1) (layer "B.Cu") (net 4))
 (segment (start 179.4462 65.783) (end 179.386 65.8432) (width 1) (layer "B.Cu") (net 4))
 (segment (start 110.1244 76.6604) (end 119.7896 76.6604) (width 1) (layer "B.Cu") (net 4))
 (segment (start 110.0074 80.7974) (end 121.7422 80.7974) (width 1) (layer "B.Cu") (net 8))
 (segment (start 107.2388 75.9206) (end 107.2388 78.0288) (width 1) (layer "B.Cu") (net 8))
 (segment (start 110.1344 74.3204) (end 108.839 74.3204) (width 1) (layer "B.Cu") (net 8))
 (segment (start 121.7422 80.7974) (end 134.112 93.1672) (width 1) (layer "B.Cu") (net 8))
 (segment (start 108.839 74.3204) (end 107.2388 75.9206) (width 1) (layer "B.Cu") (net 8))
 (segment (start 134.112 93.1672) (end 141.1732 93.1672) (width 1) (layer "B.Cu") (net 8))
 (segment (start 107.2388 78.0288) (end 110.0074 80.7974) (width 1) (layer "B.Cu") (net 8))
 (segment (start 173.2978 88.6016) (end 179.386 88.6016) (width 1) (layer "F.Cu") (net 5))
 (segment (start 179.386 88.6016) (end 157.1942 88.6016) (width 1) (layer "B.Cu") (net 5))
 (segment (start 157.1942 88.6016) (end 156.4386 89.3572) (width 1) (layer "B.Cu") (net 5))
 (segment (start 175.4822 96.3232) (end 179.386 96.3232) (width 1) (layer "F.Cu") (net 33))
 (segment (start 179.386 96.3232) (end 159.5692 96.3232) (width 1) (layer "B.Cu") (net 33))
 (segment (start 159.5692 96.3232) (end 156.4132 93.1672) (width 1) (layer "B.Cu") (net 33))
 (segment (start 182.2894 70.8216) (end 179.386 70.8216) (width 1) (layer "B.Cu") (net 42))
 (segment (start 186.676 68.323) (end 184.788 68.323) (width 1) (layer "B.Cu") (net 42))
 (segment (start 184.788 68.323) (end 182.2894 70.8216) (width 1) (layer "B.Cu") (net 42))
 (segment (start 182.2958 77.1906) (end 181.0448 78.4416) (width 1) (layer "B.Cu") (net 39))
 (segment (start 181.0448 78.4416) (end 179.386 78.4416) (width 1) (layer "B.Cu") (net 39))
 (segment (start 182.2958 72.9732) (end 182.2958 77.1906) (width 1) (layer "B.Cu") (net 39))
 (segment (start 184.406 70.863) (end 182.2958 72.9732) (width 1) (layer "B.Cu") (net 39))
 (segment (start 186.676 70.863) (end 184.406 70.863) (width 1) (layer "B.Cu") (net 39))
 (segment (start 143.1798 74.0664) (end 144.8816 75.7682) (width 1) (layer "B.Cu") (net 30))
 (segment (start 137.2362 71.2638) (end 137.2362 73.2282) (width 1) (layer "B.Cu") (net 30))
 (segment (start 137.25 71.25) (end 137.2362 71.2638) (width 1) (layer "B.Cu") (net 30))
 (segment (start 144.8816 110.8816) (end 150 116) (width 1) (layer "B.Cu") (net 30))
 (segment (start 137.2362 73.2282) (end 138.0744 74.0664) (width 1) (layer "B.Cu") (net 30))
 (segment (start 165 116) (end 177.0568 103.9432) (width 1) (layer "B.Cu") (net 30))
 (segment (start 177.0568 103.9432) (end 179.386 103.9432) (width 1) (layer "B.Cu") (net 30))
 (segment (start 144.8816 75.7682) (end 144.8816 110.8816) (width 1) (layer "B.Cu") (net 30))
 (segment (start 150 116) (end 165 116) (width 1) (layer "B.Cu") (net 30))
 (segment (start 138.0744 74.0664) (end 143.1798 74.0664) (width 1) (layer "B.Cu") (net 30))
 (segment (start 175.9712 81.5848) (end 175.9712 73.66) (width 1) (layer "B.Cu") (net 37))
 (segment (start 175.9712 73.66) (end 164.592 62.2808) (width 1) (layer "B.Cu") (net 37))
 (segment (start 144.5 69.7998) (end 144.5 71.25) (width 1) (layer "B.Cu") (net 37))
 (segment (start 179.386 83.5216) (end 177.908 83.5216) (width 1) (layer "B.Cu") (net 37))
 (segment (start 152.019 62.2808) (end 144.5 69.7998) (width 1) (layer "B.Cu") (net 37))
 (segment (start 177.908 83.5216) (end 175.9712 81.5848) (width 1) (layer "B.Cu") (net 37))
 (segment (start 164.592 62.2808) (end 152.019 62.2808) (width 1) (layer "B.Cu") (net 37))
 (segment (start 182.75 113) (end 182.75 102.4972) (width 1) (layer "B.Cu") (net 31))
 (segment (start 181.656 101.4032) (end 179.386 101.4032) (width 1) (layer "B.Cu") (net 31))
 (segment (start 141.8336 75.4888) (end 143.383 77.0382) (width 1) (layer "B.Cu") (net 31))
 (segment (start 182.75 102.4972) (end 181.656 101.4032) (width 1) (layer "B.Cu") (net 31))
 (segment (start 137.4648 75.4888) (end 141.8336 75.4888) (width 1) (layer "B.Cu") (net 31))
 (segment (start 177.5 118.25) (end 182.75 113) (width 1) (layer "B.Cu") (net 31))
 (segment (start 143.383 112.633) (end 149 118.25) (width 1) (layer "B.Cu") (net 31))
 (segment (start 135 73.024) (end 137.4648 75.4888) (width 1) (layer "B.Cu") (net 31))
 (segment (start 135 71.25) (end 135 73.024) (width 1) (layer "B.Cu") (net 31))
 (segment (start 149 118.25) (end 177.5 118.25) (width 1) (layer "B.Cu") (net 31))
 (segment (start 143.383 77.0382) (end 143.383 112.633) (width 1) (layer "B.Cu") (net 31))
 (segment (start 151.4856 60.706) (end 166.206 60.706) (width 1) (layer "B.Cu") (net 43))
 (segment (start 166.206 60.706) (end 173.8832 68.3832) (width 1) (layer "B.Cu") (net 43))
 (segment (start 142 70.1916) (end 151.4856 60.706) (width 1) (layer "B.Cu") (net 43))
 (segment (start 173.8832 68.3832) (end 179.386 68.3832) (width 1) (layer "B.Cu") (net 43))
 (segment (start 142 71.25) (end 142 70.1916) (width 1) (layer "B.Cu") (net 43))
 (segment (start 139.5 71.25) (end 139.5 69.4404) (width 1) (layer "B.Cu") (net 36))
 (segment (start 156.5656 68.7578) (end 173.8694 86.0616) (width 1) (layer "B.Cu") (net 36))
 (segment (start 156.5656 67.6148) (end 156.5656 68.7578) (width 1) (layer "B.Cu") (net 36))
 (segment (start 139.5 69.4404) (end 141.3256 67.6148) (width 1) (layer "B.Cu") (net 36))
 (segment (start 173.8694 86.0616) (end 179.386 86.0616) (width 1) (layer "B.Cu") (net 36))
 (segment (start 186.5122 95.7678) (end 186.5122 99.314) (width 1) (layer "B.Cu") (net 35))
 (segment (start 181.886 91.1416) (end 186.5122 95.7678) (width 1) (layer "B.Cu") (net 35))
 (segment (start 187.1982 100) (end 189 100) (width 1) (layer "B.Cu") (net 35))
 (segment (start 186.5122 99.314) (end 187.1982 100) (width 1) (layer "B.Cu") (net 35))
 (segment (start 179.386 91.1416) (end 181.886 91.1416) (width 1) (layer "B.Cu") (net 35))
 (segment (start 184.3786 99.6186) (end 187.3 102.54) (width 1) (layer "B.Cu") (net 34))
 (segment (start 179.386 93.7832) (end 182.6324 93.7832) (width 1) (layer "B.Cu") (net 34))
 (segment (start 184.3786 95.5294) (end 184.3786 99.6186) (width 1) (layer "B.Cu") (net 34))
 (segment (start 187.3 102.54) (end 189 102.54) (width 1) (layer "B.Cu") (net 34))
 (segment (start 182.6324 93.7832) (end 184.3786 95.5294) (width 1) (layer "B.Cu") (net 34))
 (segment (start 154.9068 64.2112) (end 153.3256 65.7924) (width 1) (layer "B.Cu") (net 10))
 (segment (start 173.8376 64.2112) (end 175.5394 62.5094) (width 1) (layer "B.Cu") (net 10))
 (segment (start 158.5976 64.2112) (end 154.9068 64.2112) (width 1) (layer "B.Cu") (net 10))
 (segment (start 175.5394 62.5094) (end 185.9424 62.5094) (width 1) (layer "B.Cu") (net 10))
 (segment (start 185.9424 62.5094) (end 186.676 63.243) (width 1) (layer "B.Cu") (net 10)))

